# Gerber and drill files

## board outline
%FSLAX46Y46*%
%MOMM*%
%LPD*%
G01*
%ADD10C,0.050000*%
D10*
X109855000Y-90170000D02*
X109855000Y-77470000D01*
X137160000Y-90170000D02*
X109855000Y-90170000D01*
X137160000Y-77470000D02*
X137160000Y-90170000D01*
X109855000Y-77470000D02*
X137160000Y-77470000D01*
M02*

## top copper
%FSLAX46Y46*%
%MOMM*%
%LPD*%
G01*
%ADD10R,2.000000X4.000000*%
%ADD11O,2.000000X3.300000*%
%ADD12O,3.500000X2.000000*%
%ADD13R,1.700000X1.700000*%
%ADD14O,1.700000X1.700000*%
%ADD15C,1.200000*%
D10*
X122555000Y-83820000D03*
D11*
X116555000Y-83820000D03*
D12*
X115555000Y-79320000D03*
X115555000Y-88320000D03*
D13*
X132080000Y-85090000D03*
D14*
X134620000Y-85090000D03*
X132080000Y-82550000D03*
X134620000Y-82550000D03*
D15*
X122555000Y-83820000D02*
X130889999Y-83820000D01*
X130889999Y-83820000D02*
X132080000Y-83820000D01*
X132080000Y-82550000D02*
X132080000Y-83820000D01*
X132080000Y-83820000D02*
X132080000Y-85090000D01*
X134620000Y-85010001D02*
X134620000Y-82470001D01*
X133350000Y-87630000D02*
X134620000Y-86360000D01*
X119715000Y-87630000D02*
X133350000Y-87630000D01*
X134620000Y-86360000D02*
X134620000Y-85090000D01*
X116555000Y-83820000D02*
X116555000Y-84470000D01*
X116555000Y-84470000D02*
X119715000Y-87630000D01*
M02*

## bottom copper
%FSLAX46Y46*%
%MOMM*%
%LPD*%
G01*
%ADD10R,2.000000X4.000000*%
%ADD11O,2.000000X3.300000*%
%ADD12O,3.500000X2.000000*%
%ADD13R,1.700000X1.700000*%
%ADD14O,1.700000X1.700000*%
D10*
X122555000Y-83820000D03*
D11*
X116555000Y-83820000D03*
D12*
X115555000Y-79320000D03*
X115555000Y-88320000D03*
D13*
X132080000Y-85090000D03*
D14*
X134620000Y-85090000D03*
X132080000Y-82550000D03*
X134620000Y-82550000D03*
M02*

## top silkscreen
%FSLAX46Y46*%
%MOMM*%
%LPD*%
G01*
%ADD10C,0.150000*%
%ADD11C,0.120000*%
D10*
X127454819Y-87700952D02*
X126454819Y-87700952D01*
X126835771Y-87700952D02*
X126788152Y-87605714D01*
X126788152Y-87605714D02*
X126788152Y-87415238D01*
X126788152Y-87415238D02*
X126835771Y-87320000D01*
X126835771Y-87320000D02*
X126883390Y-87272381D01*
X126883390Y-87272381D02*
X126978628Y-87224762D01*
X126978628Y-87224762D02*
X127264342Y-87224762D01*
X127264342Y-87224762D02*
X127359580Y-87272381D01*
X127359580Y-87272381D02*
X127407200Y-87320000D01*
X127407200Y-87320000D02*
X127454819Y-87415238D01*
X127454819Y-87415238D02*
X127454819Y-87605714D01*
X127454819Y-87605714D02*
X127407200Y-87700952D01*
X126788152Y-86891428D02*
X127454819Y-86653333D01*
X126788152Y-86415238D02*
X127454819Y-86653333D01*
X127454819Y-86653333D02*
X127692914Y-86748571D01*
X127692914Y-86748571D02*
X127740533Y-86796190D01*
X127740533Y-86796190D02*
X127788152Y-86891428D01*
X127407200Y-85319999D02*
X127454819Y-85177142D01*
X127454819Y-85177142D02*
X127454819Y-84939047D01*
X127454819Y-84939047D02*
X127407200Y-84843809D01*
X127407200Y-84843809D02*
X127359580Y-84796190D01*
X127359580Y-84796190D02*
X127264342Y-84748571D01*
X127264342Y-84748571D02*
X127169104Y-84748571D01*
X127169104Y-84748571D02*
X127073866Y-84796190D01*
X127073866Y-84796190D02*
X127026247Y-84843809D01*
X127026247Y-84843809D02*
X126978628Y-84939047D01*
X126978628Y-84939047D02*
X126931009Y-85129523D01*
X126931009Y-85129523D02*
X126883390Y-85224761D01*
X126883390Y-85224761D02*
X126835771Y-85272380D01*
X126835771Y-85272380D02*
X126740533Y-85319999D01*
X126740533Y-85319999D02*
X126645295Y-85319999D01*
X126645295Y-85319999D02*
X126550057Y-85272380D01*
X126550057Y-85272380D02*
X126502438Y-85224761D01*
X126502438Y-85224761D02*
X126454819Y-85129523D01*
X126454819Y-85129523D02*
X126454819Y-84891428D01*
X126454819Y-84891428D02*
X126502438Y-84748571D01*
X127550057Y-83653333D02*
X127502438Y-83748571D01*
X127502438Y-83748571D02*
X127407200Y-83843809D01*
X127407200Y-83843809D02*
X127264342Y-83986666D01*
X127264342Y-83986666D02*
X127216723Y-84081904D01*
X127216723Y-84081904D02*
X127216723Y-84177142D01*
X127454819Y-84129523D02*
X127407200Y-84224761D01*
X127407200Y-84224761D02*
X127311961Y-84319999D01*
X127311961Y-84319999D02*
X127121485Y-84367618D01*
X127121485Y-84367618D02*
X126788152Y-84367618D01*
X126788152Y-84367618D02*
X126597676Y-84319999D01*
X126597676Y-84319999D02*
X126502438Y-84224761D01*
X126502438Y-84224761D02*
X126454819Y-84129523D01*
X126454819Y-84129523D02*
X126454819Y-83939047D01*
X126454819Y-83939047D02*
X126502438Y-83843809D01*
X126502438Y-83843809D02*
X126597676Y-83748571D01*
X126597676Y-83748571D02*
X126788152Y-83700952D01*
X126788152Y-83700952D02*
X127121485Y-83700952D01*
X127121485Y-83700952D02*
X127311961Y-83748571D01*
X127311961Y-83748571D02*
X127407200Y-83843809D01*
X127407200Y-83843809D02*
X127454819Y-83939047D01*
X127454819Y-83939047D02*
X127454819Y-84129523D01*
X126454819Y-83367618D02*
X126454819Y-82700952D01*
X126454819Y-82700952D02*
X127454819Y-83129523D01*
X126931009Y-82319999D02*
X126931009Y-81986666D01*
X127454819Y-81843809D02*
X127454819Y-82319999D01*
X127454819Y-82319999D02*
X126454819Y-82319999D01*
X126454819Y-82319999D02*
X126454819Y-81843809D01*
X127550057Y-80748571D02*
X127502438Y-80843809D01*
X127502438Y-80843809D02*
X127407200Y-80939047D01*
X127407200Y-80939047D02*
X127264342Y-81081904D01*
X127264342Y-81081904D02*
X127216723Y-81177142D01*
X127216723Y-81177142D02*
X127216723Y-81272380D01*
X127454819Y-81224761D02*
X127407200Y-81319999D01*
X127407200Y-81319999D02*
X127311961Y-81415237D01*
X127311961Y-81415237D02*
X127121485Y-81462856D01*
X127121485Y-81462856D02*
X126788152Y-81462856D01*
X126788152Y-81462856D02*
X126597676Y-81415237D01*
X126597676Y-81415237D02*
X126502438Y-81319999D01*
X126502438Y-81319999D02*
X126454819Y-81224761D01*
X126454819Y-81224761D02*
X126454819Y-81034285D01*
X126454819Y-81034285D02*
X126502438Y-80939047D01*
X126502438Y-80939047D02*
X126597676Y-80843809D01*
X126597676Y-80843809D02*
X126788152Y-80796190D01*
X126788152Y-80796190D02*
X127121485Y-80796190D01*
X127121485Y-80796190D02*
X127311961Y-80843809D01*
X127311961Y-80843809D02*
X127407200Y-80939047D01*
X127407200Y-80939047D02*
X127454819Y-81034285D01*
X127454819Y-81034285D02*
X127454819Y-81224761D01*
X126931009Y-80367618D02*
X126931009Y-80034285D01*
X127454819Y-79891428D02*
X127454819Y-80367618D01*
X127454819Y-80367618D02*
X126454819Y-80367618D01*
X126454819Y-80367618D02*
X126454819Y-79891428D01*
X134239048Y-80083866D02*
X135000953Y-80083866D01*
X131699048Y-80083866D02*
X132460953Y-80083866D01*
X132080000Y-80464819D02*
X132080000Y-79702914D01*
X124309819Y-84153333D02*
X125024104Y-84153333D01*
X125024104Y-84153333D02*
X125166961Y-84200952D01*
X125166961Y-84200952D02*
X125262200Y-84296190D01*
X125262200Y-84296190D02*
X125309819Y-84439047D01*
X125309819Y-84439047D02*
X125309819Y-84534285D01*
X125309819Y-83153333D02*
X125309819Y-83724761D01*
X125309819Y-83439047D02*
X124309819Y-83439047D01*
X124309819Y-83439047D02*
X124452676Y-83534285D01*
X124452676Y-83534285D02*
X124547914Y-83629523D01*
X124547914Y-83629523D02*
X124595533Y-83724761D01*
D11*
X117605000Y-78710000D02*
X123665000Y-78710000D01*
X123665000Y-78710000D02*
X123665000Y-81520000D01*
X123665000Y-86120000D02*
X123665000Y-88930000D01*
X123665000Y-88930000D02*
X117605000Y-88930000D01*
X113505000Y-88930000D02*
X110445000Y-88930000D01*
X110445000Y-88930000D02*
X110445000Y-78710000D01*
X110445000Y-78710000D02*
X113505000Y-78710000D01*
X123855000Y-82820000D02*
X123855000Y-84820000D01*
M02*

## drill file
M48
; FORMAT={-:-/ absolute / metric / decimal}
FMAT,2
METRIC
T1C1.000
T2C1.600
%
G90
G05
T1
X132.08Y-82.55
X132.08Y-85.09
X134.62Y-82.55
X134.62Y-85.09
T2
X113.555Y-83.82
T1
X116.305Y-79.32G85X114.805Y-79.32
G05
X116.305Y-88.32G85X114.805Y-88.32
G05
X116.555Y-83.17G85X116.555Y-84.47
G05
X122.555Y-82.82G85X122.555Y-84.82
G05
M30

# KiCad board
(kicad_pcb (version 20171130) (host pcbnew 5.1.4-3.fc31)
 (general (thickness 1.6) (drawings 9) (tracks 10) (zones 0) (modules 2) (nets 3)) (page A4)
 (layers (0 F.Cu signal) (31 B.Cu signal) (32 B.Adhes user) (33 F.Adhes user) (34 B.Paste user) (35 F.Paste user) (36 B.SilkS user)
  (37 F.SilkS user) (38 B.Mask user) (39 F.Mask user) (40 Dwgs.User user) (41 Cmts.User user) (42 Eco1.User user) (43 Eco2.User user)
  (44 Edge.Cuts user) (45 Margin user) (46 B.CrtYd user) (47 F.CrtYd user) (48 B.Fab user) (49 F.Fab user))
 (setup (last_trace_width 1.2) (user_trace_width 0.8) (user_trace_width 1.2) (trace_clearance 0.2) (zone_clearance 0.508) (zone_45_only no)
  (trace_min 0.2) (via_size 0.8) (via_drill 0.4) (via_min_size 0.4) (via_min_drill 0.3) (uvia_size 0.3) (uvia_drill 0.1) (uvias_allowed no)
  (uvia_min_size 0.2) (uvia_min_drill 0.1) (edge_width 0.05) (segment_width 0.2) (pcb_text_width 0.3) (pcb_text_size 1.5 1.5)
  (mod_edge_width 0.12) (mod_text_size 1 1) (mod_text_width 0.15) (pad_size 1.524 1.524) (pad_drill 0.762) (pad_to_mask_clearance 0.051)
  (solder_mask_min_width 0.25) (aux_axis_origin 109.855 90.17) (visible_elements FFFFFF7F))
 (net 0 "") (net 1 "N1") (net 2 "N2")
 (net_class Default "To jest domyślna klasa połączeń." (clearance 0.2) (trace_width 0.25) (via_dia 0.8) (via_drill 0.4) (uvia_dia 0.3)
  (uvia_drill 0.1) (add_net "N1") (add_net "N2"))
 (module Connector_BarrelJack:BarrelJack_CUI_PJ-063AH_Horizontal (layer F.Cu) (at 122.555 83.82 270)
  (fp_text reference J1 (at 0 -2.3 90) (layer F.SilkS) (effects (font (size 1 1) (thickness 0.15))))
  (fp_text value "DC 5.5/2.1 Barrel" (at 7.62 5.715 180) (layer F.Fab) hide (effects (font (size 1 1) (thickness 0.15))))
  (fp_line (start -5.11 4.95) (end -5.11 -1.11) (layer F.SilkS) (width 0.12))
  (fp_line (start -5.11 -1.11) (end -2.3 -1.11) (layer F.SilkS) (width 0.12))
  (fp_line (start 2.3 -1.11) (end 5.11 -1.11) (layer F.SilkS) (width 0.12))
  (fp_line (start 5.11 -1.11) (end 5.11 4.95) (layer F.SilkS) (width 0.12))
  (fp_line (start 5.11 9.05) (end 5.11 12.11) (layer F.SilkS) (width 0.12))
  (fp_line (start 5.11 12.11) (end -5.11 12.11) (layer F.SilkS) (width 0.12))
  (fp_line (start -5.11 12.11) (end -5.11 9.05) (layer F.SilkS) (width 0.12))
  (fp_line (start -1 -1.3) (end 1 -1.3) (layer F.SilkS) (width 0.12))
  (pad 1 thru_hole rect (at 0 0 270) (size 4 2) (drill oval 3 1) (layers *.Cu *.Mask) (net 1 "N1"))
  (pad 2 thru_hole oval (at 0 6 270) (size 3.3 2) (drill oval 2.3 1) (layers *.Cu *.Mask) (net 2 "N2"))
  (pad MP thru_hole oval (at -4.5 7 270) (size 2 3.5) (drill oval 1 2.5) (layers *.Cu *.Mask))
  (pad MP thru_hole oval (at 4.5 7 270) (size 2 3.5) (drill oval 1 2.5) (layers *.Cu *.Mask))
  (pad "" np_thru_hole circle (at 0 9 270) (size 1.6 1.6) (drill 1.6) (layers *.Cu *.Mask)))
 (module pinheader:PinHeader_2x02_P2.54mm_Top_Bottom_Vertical (layer B.Cu) (at 132.08 85.09)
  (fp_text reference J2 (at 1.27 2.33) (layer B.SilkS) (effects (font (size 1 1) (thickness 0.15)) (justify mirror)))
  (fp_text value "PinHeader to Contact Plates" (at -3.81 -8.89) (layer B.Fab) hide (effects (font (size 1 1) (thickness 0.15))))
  (pad 1 thru_hole rect (at 0 0) (size 1.7 1.7) (drill 1) (layers *.Cu *.Mask) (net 1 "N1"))
  (pad 3 thru_hole oval (at 2.54 0) (size 1.7 1.7) (drill 1) (layers *.Cu *.Mask) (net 2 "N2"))
  (pad 2 thru_hole oval (at 0 -2.54) (size 1.7 1.7) (drill 1) (layers *.Cu *.Mask) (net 1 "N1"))
  (pad 4 thru_hole oval (at 2.54 -2.54) (size 1.7 1.7) (drill 1) (layers *.Cu *.Mask) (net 2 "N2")))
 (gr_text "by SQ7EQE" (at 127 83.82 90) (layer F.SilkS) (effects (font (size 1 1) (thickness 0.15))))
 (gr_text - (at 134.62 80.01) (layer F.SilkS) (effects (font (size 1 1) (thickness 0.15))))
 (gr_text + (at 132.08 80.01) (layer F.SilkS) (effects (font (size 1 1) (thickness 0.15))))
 (gr_line (start 109.855 90.17) (end 109.855 77.47) (layer Edge.Cuts) (width 0.05))
 (gr_line (start 137.16 90.17) (end 109.855 90.17) (layer Edge.Cuts) (width 0.05))
 (gr_line (start 137.16 77.47) (end 137.16 90.17) (layer Edge.Cuts) (width 0.05))
 (gr_line (start 109.855 77.47) (end 137.16 77.47) (layer Edge.Cuts) (width 0.05))
 (segment (start 122.555 83.82) (end 130.889999 83.82) (width 1.2) (layer F.Cu) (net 1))
 (segment (start 130.889999 83.82) (end 132.08 83.82) (width 1.2) (layer F.Cu) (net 1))
 (segment (start 132.08 82.55) (end 132.08 83.82) (width 1.2) (layer F.Cu) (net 1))
 (segment (start 132.08 83.82) (end 132.08 85.09) (width 1.2) (layer F.Cu) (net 1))
 (segment (start 134.62 85.010001) (end 134.62 82.470001) (width 1.2) (layer F.Cu) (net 2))
 (segment (start 133.35 87.63) (end 134.62 86.36) (width 1.2) (layer F.Cu) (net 2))
 (segment (start 119.715 87.63) (end 133.35 87.63) (width 1.2) (layer F.Cu) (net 2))
 (segment (start 134.62 86.36) (end 134.62 85.09) (width 1.2) (layer F.Cu) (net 2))
 (segment (start 116.555 83.82) (end 116.555 84.47) (width 1.2) (layer F.Cu) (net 2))
 (segment (start 116.555 84.47) (end 119.715 87.63) (width 1.2) (layer F.Cu) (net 2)))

